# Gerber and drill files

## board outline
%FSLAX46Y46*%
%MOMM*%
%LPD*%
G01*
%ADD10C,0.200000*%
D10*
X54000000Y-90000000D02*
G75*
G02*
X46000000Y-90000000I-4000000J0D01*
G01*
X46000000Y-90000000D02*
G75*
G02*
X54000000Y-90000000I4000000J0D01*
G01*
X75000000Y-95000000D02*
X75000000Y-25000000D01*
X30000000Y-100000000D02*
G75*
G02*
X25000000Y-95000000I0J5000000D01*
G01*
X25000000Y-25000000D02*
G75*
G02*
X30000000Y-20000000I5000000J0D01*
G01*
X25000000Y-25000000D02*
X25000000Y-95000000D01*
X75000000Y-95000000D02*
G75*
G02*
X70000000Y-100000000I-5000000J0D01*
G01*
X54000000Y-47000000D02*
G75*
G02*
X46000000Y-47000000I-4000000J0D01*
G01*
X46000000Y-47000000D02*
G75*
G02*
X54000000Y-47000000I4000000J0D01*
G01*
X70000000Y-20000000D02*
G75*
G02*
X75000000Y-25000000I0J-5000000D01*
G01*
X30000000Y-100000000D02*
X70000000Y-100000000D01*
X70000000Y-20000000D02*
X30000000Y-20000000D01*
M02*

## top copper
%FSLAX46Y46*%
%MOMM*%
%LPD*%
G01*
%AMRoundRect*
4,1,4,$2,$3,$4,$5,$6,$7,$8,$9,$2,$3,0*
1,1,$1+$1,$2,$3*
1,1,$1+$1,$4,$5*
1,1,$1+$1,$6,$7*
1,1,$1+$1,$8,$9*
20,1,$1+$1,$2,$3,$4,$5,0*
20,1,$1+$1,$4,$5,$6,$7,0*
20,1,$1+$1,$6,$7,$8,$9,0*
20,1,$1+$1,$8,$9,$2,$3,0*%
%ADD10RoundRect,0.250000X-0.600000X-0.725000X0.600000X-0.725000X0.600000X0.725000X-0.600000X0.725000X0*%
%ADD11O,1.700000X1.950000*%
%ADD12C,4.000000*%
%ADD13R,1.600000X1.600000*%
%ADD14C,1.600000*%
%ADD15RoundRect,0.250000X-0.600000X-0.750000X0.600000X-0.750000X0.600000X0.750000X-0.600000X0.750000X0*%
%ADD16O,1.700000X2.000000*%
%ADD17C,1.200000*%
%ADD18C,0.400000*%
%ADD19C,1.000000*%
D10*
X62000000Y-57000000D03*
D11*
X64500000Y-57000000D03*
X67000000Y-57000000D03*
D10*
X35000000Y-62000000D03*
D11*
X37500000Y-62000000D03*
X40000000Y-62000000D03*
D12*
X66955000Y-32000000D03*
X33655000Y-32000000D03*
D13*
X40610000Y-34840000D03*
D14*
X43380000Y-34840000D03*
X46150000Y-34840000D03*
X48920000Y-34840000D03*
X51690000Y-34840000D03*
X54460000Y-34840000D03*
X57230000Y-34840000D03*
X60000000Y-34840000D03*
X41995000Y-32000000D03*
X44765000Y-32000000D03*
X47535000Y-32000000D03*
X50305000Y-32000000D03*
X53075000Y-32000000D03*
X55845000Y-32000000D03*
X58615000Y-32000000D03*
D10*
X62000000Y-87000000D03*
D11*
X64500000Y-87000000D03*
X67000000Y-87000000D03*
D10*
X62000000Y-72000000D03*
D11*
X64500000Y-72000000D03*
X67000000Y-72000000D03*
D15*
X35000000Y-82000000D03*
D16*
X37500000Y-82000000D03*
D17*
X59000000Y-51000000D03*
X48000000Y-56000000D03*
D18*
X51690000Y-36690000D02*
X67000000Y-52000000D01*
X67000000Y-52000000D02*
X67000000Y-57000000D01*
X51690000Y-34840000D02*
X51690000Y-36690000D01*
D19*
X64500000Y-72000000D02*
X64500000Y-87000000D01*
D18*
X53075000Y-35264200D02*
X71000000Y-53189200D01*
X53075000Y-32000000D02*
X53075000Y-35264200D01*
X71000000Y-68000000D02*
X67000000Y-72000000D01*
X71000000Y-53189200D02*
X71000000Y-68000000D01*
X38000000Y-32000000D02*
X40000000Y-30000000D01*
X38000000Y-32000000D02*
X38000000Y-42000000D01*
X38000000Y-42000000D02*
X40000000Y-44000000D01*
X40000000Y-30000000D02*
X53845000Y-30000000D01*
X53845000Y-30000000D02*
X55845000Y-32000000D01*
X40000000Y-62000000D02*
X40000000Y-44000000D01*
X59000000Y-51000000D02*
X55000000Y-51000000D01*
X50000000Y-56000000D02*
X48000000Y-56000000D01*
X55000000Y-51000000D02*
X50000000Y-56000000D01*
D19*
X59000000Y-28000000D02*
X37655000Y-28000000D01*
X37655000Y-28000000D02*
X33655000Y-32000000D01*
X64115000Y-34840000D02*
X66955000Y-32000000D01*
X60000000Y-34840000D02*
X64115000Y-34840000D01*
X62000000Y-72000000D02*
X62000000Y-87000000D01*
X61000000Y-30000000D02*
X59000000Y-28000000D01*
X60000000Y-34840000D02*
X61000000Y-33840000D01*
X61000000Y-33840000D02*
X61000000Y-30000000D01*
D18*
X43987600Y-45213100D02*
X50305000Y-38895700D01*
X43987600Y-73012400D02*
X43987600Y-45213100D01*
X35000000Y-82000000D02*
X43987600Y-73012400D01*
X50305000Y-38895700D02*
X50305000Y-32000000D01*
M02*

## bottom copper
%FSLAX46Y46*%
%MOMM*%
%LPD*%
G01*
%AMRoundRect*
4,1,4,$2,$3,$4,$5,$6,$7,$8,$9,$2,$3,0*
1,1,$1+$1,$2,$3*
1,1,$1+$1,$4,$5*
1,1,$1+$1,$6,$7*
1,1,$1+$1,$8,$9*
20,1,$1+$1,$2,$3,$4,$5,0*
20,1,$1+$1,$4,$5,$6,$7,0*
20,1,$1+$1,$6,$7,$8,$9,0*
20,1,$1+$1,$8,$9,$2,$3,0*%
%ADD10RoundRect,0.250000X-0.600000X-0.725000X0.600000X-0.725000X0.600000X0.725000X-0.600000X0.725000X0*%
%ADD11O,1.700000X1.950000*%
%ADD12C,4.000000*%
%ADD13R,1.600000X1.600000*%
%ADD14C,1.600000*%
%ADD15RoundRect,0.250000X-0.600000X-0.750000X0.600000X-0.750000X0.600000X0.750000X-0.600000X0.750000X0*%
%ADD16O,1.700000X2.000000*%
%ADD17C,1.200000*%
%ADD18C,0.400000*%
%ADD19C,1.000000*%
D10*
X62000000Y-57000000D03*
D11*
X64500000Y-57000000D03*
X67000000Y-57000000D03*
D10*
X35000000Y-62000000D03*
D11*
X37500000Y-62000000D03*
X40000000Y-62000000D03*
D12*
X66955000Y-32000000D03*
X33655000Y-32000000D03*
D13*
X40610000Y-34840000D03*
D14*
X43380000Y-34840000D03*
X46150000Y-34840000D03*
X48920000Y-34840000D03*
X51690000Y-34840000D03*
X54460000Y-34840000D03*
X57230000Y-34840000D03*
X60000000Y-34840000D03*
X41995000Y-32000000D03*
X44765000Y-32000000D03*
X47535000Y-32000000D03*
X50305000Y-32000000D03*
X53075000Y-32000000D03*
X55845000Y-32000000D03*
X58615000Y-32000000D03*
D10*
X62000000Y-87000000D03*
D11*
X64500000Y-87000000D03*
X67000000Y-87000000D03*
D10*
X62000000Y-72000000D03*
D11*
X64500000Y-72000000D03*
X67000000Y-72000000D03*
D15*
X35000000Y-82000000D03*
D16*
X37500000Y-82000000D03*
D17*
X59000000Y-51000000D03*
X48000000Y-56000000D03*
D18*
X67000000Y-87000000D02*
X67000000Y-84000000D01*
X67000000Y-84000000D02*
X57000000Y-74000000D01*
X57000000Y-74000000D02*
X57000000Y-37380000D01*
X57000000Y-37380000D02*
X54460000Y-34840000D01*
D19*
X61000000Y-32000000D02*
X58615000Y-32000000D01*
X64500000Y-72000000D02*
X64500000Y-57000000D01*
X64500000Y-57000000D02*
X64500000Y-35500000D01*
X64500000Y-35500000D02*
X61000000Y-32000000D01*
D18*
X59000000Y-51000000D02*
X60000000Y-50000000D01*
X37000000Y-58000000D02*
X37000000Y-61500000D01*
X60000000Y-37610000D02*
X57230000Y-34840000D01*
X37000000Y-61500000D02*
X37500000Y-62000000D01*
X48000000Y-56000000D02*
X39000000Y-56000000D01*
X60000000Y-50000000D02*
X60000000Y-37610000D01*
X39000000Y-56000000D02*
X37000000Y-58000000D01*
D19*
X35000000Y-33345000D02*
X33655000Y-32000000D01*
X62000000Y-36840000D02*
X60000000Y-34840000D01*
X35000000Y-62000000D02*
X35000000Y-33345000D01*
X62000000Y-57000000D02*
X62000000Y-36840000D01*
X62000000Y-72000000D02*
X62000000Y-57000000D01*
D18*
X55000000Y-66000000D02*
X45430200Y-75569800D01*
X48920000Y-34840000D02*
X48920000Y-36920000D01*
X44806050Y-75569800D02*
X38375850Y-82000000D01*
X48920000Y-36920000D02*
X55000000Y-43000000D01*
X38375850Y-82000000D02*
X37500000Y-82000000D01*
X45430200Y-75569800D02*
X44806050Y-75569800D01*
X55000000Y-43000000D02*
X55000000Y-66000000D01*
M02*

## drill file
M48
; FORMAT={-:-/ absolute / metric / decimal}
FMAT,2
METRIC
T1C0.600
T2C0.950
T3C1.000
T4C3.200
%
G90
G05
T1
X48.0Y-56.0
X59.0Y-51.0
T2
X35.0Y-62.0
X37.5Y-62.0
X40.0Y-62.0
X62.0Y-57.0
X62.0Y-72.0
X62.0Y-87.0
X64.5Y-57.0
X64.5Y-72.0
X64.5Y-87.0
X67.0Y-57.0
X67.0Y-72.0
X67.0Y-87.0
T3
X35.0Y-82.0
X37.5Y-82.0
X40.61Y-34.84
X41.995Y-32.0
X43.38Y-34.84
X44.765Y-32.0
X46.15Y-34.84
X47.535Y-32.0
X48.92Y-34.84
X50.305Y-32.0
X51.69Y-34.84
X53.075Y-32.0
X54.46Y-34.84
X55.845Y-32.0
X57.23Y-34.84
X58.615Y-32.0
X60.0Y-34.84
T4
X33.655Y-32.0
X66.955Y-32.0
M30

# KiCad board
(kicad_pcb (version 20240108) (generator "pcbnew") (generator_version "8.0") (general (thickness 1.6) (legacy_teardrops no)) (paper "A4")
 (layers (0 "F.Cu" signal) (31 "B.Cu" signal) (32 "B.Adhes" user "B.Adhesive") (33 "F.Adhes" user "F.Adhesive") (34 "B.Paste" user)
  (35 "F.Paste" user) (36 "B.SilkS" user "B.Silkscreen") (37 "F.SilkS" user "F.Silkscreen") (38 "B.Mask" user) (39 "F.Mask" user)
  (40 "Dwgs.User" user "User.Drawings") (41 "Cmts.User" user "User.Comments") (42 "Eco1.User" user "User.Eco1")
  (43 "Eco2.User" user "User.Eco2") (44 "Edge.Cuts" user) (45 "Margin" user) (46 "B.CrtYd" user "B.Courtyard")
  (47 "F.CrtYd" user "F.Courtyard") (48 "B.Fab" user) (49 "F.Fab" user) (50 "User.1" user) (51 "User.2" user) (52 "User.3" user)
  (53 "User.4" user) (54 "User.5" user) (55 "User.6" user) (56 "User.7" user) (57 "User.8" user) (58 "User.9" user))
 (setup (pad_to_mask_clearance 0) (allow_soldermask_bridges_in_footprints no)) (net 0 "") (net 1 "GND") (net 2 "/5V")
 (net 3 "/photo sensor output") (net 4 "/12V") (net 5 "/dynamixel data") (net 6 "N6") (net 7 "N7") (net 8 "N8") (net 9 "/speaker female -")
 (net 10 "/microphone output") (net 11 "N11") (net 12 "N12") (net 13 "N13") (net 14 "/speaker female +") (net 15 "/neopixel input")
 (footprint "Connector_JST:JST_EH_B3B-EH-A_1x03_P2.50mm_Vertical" (layer "F.Cu") (at 62 57)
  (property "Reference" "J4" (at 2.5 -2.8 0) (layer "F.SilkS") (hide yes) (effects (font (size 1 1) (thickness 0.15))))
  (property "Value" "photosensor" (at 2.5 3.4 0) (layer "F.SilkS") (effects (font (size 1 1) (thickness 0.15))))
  (pad "1" thru_hole roundrect (at 0 0) (size 1.7 1.95) (drill 0.95) (layers "*.Cu" "*.Mask") (remove_unused_layers no)
   (roundrect_rratio 0.147059) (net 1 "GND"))
  (pad "2" thru_hole oval (at 2.5 0) (size 1.7 1.95) (drill 0.95) (layers "*.Cu" "*.Mask") (remove_unused_layers no) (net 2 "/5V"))
  (pad "3" thru_hole oval (at 5 0) (size 1.7 1.95) (drill 0.95) (layers "*.Cu" "*.Mask") (remove_unused_layers no)
   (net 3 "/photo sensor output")))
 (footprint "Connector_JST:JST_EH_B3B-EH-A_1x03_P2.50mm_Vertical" (layer "F.Cu") (at 35 62)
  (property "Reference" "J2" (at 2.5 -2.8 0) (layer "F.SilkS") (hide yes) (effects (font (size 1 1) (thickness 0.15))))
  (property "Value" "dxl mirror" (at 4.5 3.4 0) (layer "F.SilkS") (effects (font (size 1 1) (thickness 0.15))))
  (pad "1" thru_hole roundrect (at 0 0) (size 1.7 1.95) (drill 0.95) (layers "*.Cu" "*.Mask") (remove_unused_layers no)
   (roundrect_rratio 0.147059) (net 1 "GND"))
  (pad "2" thru_hole oval (at 2.5 0) (size 1.7 1.95) (drill 0.95) (layers "*.Cu" "*.Mask") (remove_unused_layers no) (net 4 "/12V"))
  (pad "3" thru_hole oval (at 5 0) (size 1.7 1.95) (drill 0.95) (layers "*.Cu" "*.Mask") (remove_unused_layers no) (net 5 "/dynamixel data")))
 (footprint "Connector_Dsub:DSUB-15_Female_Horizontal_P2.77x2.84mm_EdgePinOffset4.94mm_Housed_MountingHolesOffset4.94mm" (layer "F.Cu")
  (at 40.61 34.84 180)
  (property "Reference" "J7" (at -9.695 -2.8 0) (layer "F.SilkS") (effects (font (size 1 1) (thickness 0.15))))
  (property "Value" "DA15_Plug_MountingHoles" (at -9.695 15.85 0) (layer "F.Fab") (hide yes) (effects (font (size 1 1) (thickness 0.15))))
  (pad "0" thru_hole circle (at -26.345 2.84 180) (size 4 4) (drill 3.2) (layers "*.Cu" "*.Mask") (remove_unused_layers no) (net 1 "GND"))
  (pad "0" thru_hole circle (at 6.955 2.84 180) (size 4 4) (drill 3.2) (layers "*.Cu" "*.Mask") (remove_unused_layers no) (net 1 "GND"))
  (pad "1" thru_hole rect (at 0 0 180) (size 1.6 1.6) (drill 1) (layers "*.Cu" "*.Mask") (remove_unused_layers no) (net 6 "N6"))
  (pad "2" thru_hole circle (at -2.77 0 180) (size 1.6 1.6) (drill 1) (layers "*.Cu" "*.Mask") (remove_unused_layers no) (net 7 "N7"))
  (pad "3" thru_hole circle (at -5.54 0 180) (size 1.6 1.6) (drill 1) (layers "*.Cu" "*.Mask") (remove_unused_layers no) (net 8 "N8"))
  (pad "4" thru_hole circle (at -8.31 0 180) (size 1.6 1.6) (drill 1) (layers "*.Cu" "*.Mask") (remove_unused_layers no)
   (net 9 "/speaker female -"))
  (pad "5" thru_hole circle (at -11.08 0 180) (size 1.6 1.6) (drill 1) (layers "*.Cu" "*.Mask") (remove_unused_layers no)
   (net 3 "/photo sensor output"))
  (pad "6" thru_hole circle (at -13.85 0 180) (size 1.6 1.6) (drill 1) (layers "*.Cu" "*.Mask") (remove_unused_layers no)
   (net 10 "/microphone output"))
  (pad "7" thru_hole circle (at -16.62 0 180) (size 1.6 1.6) (drill 1) (layers "*.Cu" "*.Mask") (remove_unused_layers no) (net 4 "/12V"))
  (pad "8" thru_hole circle (at -19.39 0 180) (size 1.6 1.6) (drill 1) (layers "*.Cu" "*.Mask") (remove_unused_layers no) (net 1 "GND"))
  (pad "9" thru_hole circle (at -1.385 2.84 180) (size 1.6 1.6) (drill 1) (layers "*.Cu" "*.Mask") (remove_unused_layers no) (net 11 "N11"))
  (pad "10" thru_hole circle (at -4.155 2.84 180) (size 1.6 1.6) (drill 1) (layers "*.Cu" "*.Mask") (remove_unused_layers no) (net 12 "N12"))
  (pad "11" thru_hole circle (at -6.925 2.84 180) (size 1.6 1.6) (drill 1) (layers "*.Cu" "*.Mask") (remove_unused_layers no) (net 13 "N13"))
  (pad "12" thru_hole circle (at -9.695 2.84 180) (size 1.6 1.6) (drill 1) (layers "*.Cu" "*.Mask") (remove_unused_layers no)
   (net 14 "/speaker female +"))
  (pad "13" thru_hole circle (at -12.465 2.84 180) (size 1.6 1.6) (drill 1) (layers "*.Cu" "*.Mask") (remove_unused_layers no)
   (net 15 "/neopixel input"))
  (pad "14" thru_hole circle (at -15.235 2.84 180) (size 1.6 1.6) (drill 1) (layers "*.Cu" "*.Mask") (remove_unused_layers no)
   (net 5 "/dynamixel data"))
  (pad "15" thru_hole circle (at -18.005 2.84 180) (size 1.6 1.6) (drill 1) (layers "*.Cu" "*.Mask") (remove_unused_layers no) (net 2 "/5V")))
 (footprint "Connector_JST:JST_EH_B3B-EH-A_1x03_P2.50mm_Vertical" (layer "F.Cu") (at 62 87)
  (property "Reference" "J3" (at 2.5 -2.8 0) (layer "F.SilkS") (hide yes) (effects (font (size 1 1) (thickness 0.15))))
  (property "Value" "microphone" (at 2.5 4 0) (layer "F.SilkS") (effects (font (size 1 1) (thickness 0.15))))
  (pad "1" thru_hole roundrect (at 0 0) (size 1.7 1.95) (drill 0.95) (layers "*.Cu" "*.Mask") (remove_unused_layers no)
   (roundrect_rratio 0.147059) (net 1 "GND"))
  (pad "2" thru_hole oval (at 2.5 0) (size 1.7 1.95) (drill 0.95) (layers "*.Cu" "*.Mask") (remove_unused_layers no) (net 2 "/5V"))
  (pad "3" thru_hole oval (at 5 0) (size 1.7 1.95) (drill 0.95) (layers "*.Cu" "*.Mask") (remove_unused_layers no)
   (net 10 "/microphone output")))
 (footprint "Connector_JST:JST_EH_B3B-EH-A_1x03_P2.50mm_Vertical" (layer "F.Cu") (at 62 72)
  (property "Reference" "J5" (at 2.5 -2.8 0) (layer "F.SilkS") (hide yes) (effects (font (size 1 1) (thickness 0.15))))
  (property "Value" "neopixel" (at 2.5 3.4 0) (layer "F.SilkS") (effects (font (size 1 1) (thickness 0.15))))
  (pad "1" thru_hole roundrect (at 0 0) (size 1.7 1.95) (drill 0.95) (layers "*.Cu" "*.Mask") (remove_unused_layers no)
   (roundrect_rratio 0.147059) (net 1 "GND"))
  (pad "2" thru_hole oval (at 2.5 0) (size 1.7 1.95) (drill 0.95) (layers "*.Cu" "*.Mask") (remove_unused_layers no) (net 2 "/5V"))
  (pad "3" thru_hole oval (at 5 0) (size 1.7 1.95) (drill 0.95) (layers "*.Cu" "*.Mask") (remove_unused_layers no)
   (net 15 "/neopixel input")))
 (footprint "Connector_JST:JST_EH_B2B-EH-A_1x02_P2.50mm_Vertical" (layer "F.Cu") (at 35 82)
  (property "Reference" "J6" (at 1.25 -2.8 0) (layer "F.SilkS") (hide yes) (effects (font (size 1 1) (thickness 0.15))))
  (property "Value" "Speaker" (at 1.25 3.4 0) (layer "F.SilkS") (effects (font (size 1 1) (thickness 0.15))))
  (pad "1" thru_hole roundrect (at 0 0) (size 1.7 2) (drill 1) (layers "*.Cu" "*.Mask") (remove_unused_layers no)
   (roundrect_rratio 0.147059) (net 14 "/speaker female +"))
  (pad "2" thru_hole oval (at 2.5 0) (size 1.7 2) (drill 1) (layers "*.Cu" "*.Mask") (remove_unused_layers no) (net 9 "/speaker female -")))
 (gr_circle (center 50 90) (end 54 90) (stroke (width 0.2) (type default)) (fill none) (layer "Edge.Cuts"))
 (gr_line (start 75 95) (end 75 25) (stroke (width 0.2) (type default)) (layer "Edge.Cuts"))
 (gr_arc (start 30 100) (mid 26.464466 98.535534) (end 25 95) (stroke (width 0.2) (type default)) (layer "Edge.Cuts"))
 (gr_arc (start 25 25) (mid 26.464466 21.464466) (end 30 20) (stroke (width 0.2) (type default)) (layer "Edge.Cuts"))
 (gr_line (start 25 25) (end 25 95) (stroke (width 0.2) (type default)) (layer "Edge.Cuts"))
 (gr_arc (start 75 95) (mid 73.535534 98.535534) (end 70 100) (stroke (width 0.2) (type default)) (layer "Edge.Cuts"))
 (gr_circle (center 50 47) (end 54 47) (stroke (width 0.2) (type default)) (fill none) (layer "Edge.Cuts"))
 (gr_arc (start 70 20) (mid 73.535534 21.464466) (end 75 25) (stroke (width 0.2) (type default)) (layer "Edge.Cuts"))
 (gr_line (start 30 100) (end 70 100) (stroke (width 0.2) (type default)) (layer "Edge.Cuts"))
 (gr_line (start 70 20) (end 30 20) (stroke (width 0.2) (type default)) (layer "Edge.Cuts"))
 (segment (start 51.69 36.69) (end 67 52) (width 0.4) (layer "F.Cu") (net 3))
 (segment (start 67 52) (end 67 57) (width 0.4) (layer "F.Cu") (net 3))
 (segment (start 51.69 34.84) (end 51.69 36.69) (width 0.4) (layer "F.Cu") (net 3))
 (segment (start 67 87) (end 67 84) (width 0.4) (layer "B.Cu") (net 10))
 (segment (start 67 84) (end 57 74) (width 0.4) (layer "B.Cu") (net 10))
 (segment (start 57 74) (end 57 37.38) (width 0.4) (layer "B.Cu") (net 10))
 (segment (start 57 37.38) (end 54.46 34.84) (width 0.4) (layer "B.Cu") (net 10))
 (segment (start 64.5 72) (end 64.5 87) (width 1) (layer "F.Cu") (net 2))
 (segment (start 61 32) (end 58.615 32) (width 1) (layer "B.Cu") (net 2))
 (segment (start 64.5 72) (end 64.5 57) (width 1) (layer "B.Cu") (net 2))
 (segment (start 64.5 57) (end 64.5 35.5) (width 1) (layer "B.Cu") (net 2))
 (segment (start 64.5 35.5) (end 61 32) (width 1) (layer "B.Cu") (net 2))
 (segment (start 53.075 35.2642) (end 71 53.1892) (width 0.4) (layer "F.Cu") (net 15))
 (segment (start 53.075 32) (end 53.075 35.2642) (width 0.4) (layer "F.Cu") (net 15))
 (segment (start 71 68) (end 67 72) (width 0.4) (layer "F.Cu") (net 15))
 (segment (start 71 53.1892) (end 71 68) (width 0.4) (layer "F.Cu") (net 15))
 (segment (start 38 32) (end 40 30) (width 0.4) (layer "F.Cu") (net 5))
 (segment (start 38 32) (end 38 42) (width 0.4) (layer "F.Cu") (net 5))
 (segment (start 38 42) (end 40 44) (width 0.4) (layer "F.Cu") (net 5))
 (segment (start 40 30) (end 53.845 30) (width 0.4) (layer "F.Cu") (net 5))
 (segment (start 53.845 30) (end 55.845 32) (width 0.4) (layer "F.Cu") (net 5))
 (segment (start 40 62) (end 40 44) (width 0.4) (layer "F.Cu") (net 5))
 (segment (start 59 51) (end 55 51) (width 0.4) (layer "F.Cu") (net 4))
 (segment (start 50 56) (end 48 56) (width 0.4) (layer "F.Cu") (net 4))
 (segment (start 55 51) (end 50 56) (width 0.4) (layer "F.Cu") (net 4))
 (via (at 59 51) (size 1.2) (drill 0.6) (layers "F.Cu" "B.Cu") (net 4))
 (via (at 48 56) (size 1.2) (drill 0.6) (layers "F.Cu" "B.Cu") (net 4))
 (segment (start 59 51) (end 60 50) (width 0.4) (layer "B.Cu") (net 4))
 (segment (start 37 58) (end 37 61.5) (width 0.4) (layer "B.Cu") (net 4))
 (segment (start 60 37.61) (end 57.23 34.84) (width 0.4) (layer "B.Cu") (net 4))
 (segment (start 37 61.5) (end 37.5 62) (width 0.4) (layer "B.Cu") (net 4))
 (segment (start 48 56) (end 39 56) (width 0.4) (layer "B.Cu") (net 4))
 (segment (start 60 50) (end 60 37.61) (width 0.4) (layer "B.Cu") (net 4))
 (segment (start 39 56) (end 37 58) (width 0.4) (layer "B.Cu") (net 4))
 (segment (start 59 28) (end 37.655 28) (width 1) (layer "F.Cu") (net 1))
 (segment (start 37.655 28) (end 33.655 32) (width 1) (layer "F.Cu") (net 1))
 (segment (start 64.115 34.84) (end 66.955 32) (width 1) (layer "F.Cu") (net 1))
 (segment (start 60 34.84) (end 64.115 34.84) (width 1) (layer "F.Cu") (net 1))
 (segment (start 62 72) (end 62 87) (width 1) (layer "F.Cu") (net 1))
 (segment (start 61 30) (end 59 28) (width 1) (layer "F.Cu") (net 1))
 (segment (start 60 34.84) (end 61 33.84) (width 1) (layer "F.Cu") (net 1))
 (segment (start 61 33.84) (end 61 30) (width 1) (layer "F.Cu") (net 1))
 (segment (start 35 33.345) (end 33.655 32) (width 1) (layer "B.Cu") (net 1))
 (segment (start 62 36.84) (end 60 34.84) (width 1) (layer "B.Cu") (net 1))
 (segment (start 35 62) (end 35 33.345) (width 1) (layer "B.Cu") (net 1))
 (segment (start 62 57) (end 62 36.84) (width 1) (layer "B.Cu") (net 1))
 (segment (start 62 72) (end 62 57) (width 1) (layer "B.Cu") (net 1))
 (segment (start 43.9876 45.2131) (end 50.305 38.8957) (width 0.4) (layer "F.Cu") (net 14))
 (segment (start 43.9876 73.0124) (end 43.9876 45.2131) (width 0.4) (layer "F.Cu") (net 14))
 (segment (start 35 82) (end 43.9876 73.0124) (width 0.4) (layer "F.Cu") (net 14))
 (segment (start 50.305 38.8957) (end 50.305 32) (width 0.4) (layer "F.Cu") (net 14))
 (segment (start 55 66) (end 45.4302 75.5698) (width 0.4) (layer "B.Cu") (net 9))
 (segment (start 48.92 34.84) (end 48.92 36.92) (width 0.4) (layer "B.Cu") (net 9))
 (segment (start 44.80605 75.5698) (end 38.37585 82) (width 0.4) (layer "B.Cu") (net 9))
 (segment (start 48.92 36.92) (end 55 43) (width 0.4) (layer "B.Cu") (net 9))
 (segment (start 38.37585 82) (end 37.5 82) (width 0.4) (layer "B.Cu") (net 9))
 (segment (start 45.4302 75.5698) (end 44.80605 75.5698) (width 0.4) (layer "B.Cu") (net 9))
 (segment (start 55 43) (end 55 66) (width 0.4) (layer "B.Cu") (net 9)))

